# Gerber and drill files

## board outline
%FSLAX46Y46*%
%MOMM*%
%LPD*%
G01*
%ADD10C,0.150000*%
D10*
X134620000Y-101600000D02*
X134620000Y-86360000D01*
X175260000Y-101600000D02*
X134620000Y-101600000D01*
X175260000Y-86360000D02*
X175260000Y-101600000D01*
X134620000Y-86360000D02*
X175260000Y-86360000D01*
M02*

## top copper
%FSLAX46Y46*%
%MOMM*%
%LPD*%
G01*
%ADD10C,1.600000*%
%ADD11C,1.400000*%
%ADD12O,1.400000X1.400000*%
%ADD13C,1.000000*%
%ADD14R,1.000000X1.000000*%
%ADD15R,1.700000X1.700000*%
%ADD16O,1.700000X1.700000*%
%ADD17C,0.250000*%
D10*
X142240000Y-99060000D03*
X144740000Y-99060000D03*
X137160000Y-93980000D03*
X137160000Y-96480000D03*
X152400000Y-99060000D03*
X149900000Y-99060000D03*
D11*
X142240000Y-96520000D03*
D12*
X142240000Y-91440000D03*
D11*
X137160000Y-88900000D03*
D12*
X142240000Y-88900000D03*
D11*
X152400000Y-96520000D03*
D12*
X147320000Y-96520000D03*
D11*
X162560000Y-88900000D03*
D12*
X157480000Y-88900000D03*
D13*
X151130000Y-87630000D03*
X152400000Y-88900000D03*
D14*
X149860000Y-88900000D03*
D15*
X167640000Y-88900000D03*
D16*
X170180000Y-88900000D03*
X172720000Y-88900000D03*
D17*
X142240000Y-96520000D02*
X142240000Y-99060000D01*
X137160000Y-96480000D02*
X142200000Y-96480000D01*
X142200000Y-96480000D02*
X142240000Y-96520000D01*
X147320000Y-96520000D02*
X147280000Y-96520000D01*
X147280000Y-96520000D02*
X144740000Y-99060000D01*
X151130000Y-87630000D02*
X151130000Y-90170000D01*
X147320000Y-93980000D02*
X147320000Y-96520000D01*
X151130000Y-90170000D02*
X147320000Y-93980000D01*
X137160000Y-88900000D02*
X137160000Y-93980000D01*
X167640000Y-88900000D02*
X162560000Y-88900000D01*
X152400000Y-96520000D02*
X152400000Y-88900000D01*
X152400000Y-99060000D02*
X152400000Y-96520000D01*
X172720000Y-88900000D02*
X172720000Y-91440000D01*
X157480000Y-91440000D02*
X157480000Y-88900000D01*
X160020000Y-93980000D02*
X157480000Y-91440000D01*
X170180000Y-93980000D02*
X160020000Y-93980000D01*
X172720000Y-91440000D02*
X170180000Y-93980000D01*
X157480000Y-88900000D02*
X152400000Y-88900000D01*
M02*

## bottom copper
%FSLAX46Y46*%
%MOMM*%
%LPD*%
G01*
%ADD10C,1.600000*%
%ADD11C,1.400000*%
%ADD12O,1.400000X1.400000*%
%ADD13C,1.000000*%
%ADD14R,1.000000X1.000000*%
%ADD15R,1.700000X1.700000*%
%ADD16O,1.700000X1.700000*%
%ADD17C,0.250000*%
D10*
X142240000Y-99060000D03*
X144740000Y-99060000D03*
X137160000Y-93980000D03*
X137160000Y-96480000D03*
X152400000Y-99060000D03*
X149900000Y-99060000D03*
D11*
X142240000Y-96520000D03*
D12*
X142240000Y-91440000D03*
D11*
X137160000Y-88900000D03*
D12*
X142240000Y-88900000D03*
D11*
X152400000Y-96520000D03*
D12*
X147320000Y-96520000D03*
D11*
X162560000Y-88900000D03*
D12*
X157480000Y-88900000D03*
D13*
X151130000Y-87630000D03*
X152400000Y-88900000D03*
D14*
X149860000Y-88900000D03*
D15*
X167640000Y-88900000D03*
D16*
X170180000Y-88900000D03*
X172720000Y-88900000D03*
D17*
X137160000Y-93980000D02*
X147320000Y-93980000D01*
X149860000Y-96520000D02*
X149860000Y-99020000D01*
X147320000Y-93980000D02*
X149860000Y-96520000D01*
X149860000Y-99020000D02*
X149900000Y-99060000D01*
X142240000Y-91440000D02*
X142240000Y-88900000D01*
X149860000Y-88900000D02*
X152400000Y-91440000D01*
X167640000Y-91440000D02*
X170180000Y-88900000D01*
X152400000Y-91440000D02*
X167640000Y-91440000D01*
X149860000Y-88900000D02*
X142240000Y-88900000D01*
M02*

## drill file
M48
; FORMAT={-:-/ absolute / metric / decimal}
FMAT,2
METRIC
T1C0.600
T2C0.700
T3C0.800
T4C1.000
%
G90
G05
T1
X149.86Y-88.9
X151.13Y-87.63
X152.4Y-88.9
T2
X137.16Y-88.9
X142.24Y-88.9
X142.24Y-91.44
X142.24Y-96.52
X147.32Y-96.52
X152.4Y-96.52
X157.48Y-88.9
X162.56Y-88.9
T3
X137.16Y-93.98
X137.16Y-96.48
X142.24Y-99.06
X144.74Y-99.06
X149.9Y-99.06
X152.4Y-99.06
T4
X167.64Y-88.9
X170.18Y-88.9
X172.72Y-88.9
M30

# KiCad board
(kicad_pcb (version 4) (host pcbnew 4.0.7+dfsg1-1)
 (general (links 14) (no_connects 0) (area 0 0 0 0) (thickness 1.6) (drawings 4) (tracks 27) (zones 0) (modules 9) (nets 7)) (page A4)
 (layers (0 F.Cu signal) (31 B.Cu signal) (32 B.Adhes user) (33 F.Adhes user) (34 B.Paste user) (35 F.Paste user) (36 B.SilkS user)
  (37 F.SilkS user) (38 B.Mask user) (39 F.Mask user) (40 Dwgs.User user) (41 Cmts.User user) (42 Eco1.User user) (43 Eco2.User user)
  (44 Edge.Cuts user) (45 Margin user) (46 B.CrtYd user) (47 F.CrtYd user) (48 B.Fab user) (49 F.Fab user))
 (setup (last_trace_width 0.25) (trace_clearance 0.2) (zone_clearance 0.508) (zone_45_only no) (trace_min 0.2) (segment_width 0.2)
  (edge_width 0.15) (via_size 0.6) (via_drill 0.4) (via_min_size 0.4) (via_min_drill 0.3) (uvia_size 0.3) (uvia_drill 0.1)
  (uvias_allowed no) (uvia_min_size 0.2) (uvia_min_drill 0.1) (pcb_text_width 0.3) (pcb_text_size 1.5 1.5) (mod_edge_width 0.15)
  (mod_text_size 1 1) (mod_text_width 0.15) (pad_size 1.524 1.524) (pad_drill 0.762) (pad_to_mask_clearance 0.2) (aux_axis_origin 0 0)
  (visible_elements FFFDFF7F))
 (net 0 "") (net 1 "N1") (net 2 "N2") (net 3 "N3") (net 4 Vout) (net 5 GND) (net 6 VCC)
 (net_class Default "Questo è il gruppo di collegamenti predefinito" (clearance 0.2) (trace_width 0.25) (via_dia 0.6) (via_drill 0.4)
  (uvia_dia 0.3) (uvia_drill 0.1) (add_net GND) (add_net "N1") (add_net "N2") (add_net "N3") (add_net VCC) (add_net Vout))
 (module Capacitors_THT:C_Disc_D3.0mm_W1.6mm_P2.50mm (layer F.Cu) (at 142.24 99.06)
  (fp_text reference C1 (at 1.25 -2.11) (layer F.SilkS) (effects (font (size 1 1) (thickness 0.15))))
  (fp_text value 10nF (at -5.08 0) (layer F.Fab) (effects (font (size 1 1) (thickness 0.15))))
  (pad 1 thru_hole circle (at 0 0) (size 1.6 1.6) (drill 0.8) (layers *.Cu *.Mask) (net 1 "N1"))
  (pad 2 thru_hole circle (at 2.5 0) (size 1.6 1.6) (drill 0.8) (layers *.Cu *.Mask) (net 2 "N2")))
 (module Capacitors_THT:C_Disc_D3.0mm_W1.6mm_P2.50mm (layer F.Cu) (at 137.16 93.98 270)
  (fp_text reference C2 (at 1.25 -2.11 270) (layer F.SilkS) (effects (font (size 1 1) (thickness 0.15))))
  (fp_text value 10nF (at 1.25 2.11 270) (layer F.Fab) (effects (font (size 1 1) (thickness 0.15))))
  (pad 1 thru_hole circle (at 0 0 270) (size 1.6 1.6) (drill 0.8) (layers *.Cu *.Mask) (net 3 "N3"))
  (pad 2 thru_hole circle (at 2.5 0 270) (size 1.6 1.6) (drill 0.8) (layers *.Cu *.Mask) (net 1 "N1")))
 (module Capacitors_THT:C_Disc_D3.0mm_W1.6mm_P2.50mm (layer F.Cu) (at 152.4 99.06 180)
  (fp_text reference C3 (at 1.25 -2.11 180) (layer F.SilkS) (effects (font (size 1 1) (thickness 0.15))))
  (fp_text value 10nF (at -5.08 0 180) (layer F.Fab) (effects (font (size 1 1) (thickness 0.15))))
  (pad 1 thru_hole circle (at 0 0 180) (size 1.6 1.6) (drill 0.8) (layers *.Cu *.Mask) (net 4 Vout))
  (pad 2 thru_hole circle (at 2.5 0 180) (size 1.6 1.6) (drill 0.8) (layers *.Cu *.Mask) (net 3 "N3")))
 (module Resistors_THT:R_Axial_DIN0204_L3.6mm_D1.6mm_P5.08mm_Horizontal (layer F.Cu) (at 142.24 96.52 90)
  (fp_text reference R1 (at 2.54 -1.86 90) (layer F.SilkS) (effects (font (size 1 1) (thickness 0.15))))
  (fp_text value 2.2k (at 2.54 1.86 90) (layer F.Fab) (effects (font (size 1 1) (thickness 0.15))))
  (pad 1 thru_hole circle (at 0 0 90) (size 1.4 1.4) (drill 0.7) (layers *.Cu *.Mask) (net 1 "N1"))
  (pad 2 thru_hole oval (at 5.08 0 90) (size 1.4 1.4) (drill 0.7) (layers *.Cu *.Mask) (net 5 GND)))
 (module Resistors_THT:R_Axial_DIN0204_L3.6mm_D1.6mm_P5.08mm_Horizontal (layer F.Cu) (at 137.16 88.9)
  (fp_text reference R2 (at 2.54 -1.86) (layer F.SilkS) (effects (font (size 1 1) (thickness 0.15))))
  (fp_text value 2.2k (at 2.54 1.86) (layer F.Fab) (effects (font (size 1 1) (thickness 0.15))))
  (pad 1 thru_hole circle (at 0 0) (size 1.4 1.4) (drill 0.7) (layers *.Cu *.Mask) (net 3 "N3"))
  (pad 2 thru_hole oval (at 5.08 0) (size 1.4 1.4) (drill 0.7) (layers *.Cu *.Mask) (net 5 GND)))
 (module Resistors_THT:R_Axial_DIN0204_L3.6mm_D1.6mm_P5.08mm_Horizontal (layer F.Cu) (at 152.4 96.52 180)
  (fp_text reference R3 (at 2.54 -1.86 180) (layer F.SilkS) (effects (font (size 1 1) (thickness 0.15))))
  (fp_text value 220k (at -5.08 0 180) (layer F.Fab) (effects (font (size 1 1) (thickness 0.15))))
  (pad 1 thru_hole circle (at 0 0 180) (size 1.4 1.4) (drill 0.7) (layers *.Cu *.Mask) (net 4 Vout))
  (pad 2 thru_hole oval (at 5.08 0 180) (size 1.4 1.4) (drill 0.7) (layers *.Cu *.Mask) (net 2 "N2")))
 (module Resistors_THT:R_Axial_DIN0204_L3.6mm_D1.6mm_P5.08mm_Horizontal (layer F.Cu) (at 162.56 88.9 180)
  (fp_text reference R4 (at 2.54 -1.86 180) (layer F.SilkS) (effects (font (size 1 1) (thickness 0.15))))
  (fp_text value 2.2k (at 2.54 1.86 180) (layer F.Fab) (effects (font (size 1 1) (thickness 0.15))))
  (pad 1 thru_hole circle (at 0 0 180) (size 1.4 1.4) (drill 0.7) (layers *.Cu *.Mask) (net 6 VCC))
  (pad 2 thru_hole oval (at 5.08 0 180) (size 1.4 1.4) (drill 0.7) (layers *.Cu *.Mask) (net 4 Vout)))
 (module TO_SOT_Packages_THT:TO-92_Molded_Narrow (layer F.Cu) (at 149.86 88.9)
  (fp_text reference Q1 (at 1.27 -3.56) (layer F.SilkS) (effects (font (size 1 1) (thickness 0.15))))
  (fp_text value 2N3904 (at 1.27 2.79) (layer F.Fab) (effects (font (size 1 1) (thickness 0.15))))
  (pad 2 thru_hole circle (at 1.27 -1.27 90) (size 1 1) (drill 0.6) (layers *.Cu *.Mask) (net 2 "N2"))
  (pad 3 thru_hole circle (at 2.54 0 90) (size 1 1) (drill 0.6) (layers *.Cu *.Mask) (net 4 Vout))
  (pad 1 thru_hole rect (at 0 0 90) (size 1 1) (drill 0.6) (layers *.Cu *.Mask) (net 5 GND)))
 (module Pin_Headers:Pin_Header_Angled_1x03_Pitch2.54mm (layer F.Cu) (at 167.64 88.9 90)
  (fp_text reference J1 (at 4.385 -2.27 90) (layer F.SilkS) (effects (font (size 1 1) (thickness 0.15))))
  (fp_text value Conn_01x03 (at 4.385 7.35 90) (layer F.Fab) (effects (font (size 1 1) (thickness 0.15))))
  (pad 1 thru_hole rect (at 0 0 90) (size 1.7 1.7) (drill 1) (layers *.Cu *.Mask) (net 6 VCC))
  (pad 2 thru_hole oval (at 0 2.54 90) (size 1.7 1.7) (drill 1) (layers *.Cu *.Mask) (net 5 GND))
  (pad 3 thru_hole oval (at 0 5.08 90) (size 1.7 1.7) (drill 1) (layers *.Cu *.Mask) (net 4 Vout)))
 (gr_line (start 134.62 101.6) (end 134.62 86.36) (angle 90) (layer Edge.Cuts) (width 0.15))
 (gr_line (start 175.26 101.6) (end 134.62 101.6) (angle 90) (layer Edge.Cuts) (width 0.15))
 (gr_line (start 175.26 86.36) (end 175.26 101.6) (angle 90) (layer Edge.Cuts) (width 0.15))
 (gr_line (start 134.62 86.36) (end 175.26 86.36) (angle 90) (layer Edge.Cuts) (width 0.15))
 (segment (start 142.24 96.52) (end 142.24 99.06) (width 0.25) (layer F.Cu) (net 1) (status C00000))
 (segment (start 137.16 96.48) (end 142.2 96.48) (width 0.25) (layer F.Cu) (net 1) (status C00000))
 (segment (start 142.2 96.48) (end 142.24 96.52) (width 0.25) (layer F.Cu) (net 1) (status C00000))
 (segment (start 147.32 96.52) (end 147.28 96.52) (width 0.25) (layer F.Cu) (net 2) (status C00000))
 (segment (start 147.28 96.52) (end 144.74 99.06) (width 0.25) (layer F.Cu) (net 2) (status C00000))
 (segment (start 151.13 87.63) (end 151.13 90.17) (width 0.25) (layer F.Cu) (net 2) (status 400000))
 (segment (start 147.32 93.98) (end 147.32 96.52) (width 0.25) (layer F.Cu) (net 2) (status 800000))
 (segment (start 151.13 90.17) (end 147.32 93.98) (width 0.25) (layer F.Cu) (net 2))
 (segment (start 137.16 93.98) (end 147.32 93.98) (width 0.25) (layer B.Cu) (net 3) (status 400000))
 (segment (start 149.86 96.52) (end 149.86 99.02) (width 0.25) (layer B.Cu) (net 3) (status 800000))
 (segment (start 147.32 93.98) (end 149.86 96.52) (width 0.25) (layer B.Cu) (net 3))
 (segment (start 149.86 99.02) (end 149.9 99.06) (width 0.25) (layer B.Cu) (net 3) (status C00000))
 (segment (start 137.16 88.9) (end 137.16 93.98) (width 0.25) (layer F.Cu) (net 3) (status C00000))
 (segment (start 142.24 91.44) (end 142.24 88.9) (width 0.25) (layer B.Cu) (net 5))
 (segment (start 149.86 88.9) (end 152.4 91.44) (width 0.25) (layer B.Cu) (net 5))
 (segment (start 167.64 91.44) (end 170.18 88.9) (width 0.25) (layer B.Cu) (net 5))
 (segment (start 152.4 91.44) (end 167.64 91.44) (width 0.25) (layer B.Cu) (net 5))
 (segment (start 149.86 88.9) (end 142.24 88.9) (width 0.25) (layer B.Cu) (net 5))
 (segment (start 167.64 88.9) (end 162.56 88.9) (width 0.25) (layer F.Cu) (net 6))
 (segment (start 152.4 96.52) (end 152.4 88.9) (width 0.25) (layer F.Cu) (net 4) (status C00000))
 (segment (start 152.4 99.06) (end 152.4 96.52) (width 0.25) (layer F.Cu) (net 4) (status C00000))
 (segment (start 172.72 88.9) (end 172.72 91.44) (width 0.25) (layer F.Cu) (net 4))
 (segment (start 157.48 91.44) (end 157.48 88.9) (width 0.25) (layer F.Cu) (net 4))
 (segment (start 160.02 93.98) (end 157.48 91.44) (width 0.25) (layer F.Cu) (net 4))
 (segment (start 170.18 93.98) (end 160.02 93.98) (width 0.25) (layer F.Cu) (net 4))
 (segment (start 172.72 91.44) (end 170.18 93.98) (width 0.25) (layer F.Cu) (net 4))
 (segment (start 157.48 88.9) (end 152.4 88.9) (width 0.25) (layer F.Cu) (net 4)))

